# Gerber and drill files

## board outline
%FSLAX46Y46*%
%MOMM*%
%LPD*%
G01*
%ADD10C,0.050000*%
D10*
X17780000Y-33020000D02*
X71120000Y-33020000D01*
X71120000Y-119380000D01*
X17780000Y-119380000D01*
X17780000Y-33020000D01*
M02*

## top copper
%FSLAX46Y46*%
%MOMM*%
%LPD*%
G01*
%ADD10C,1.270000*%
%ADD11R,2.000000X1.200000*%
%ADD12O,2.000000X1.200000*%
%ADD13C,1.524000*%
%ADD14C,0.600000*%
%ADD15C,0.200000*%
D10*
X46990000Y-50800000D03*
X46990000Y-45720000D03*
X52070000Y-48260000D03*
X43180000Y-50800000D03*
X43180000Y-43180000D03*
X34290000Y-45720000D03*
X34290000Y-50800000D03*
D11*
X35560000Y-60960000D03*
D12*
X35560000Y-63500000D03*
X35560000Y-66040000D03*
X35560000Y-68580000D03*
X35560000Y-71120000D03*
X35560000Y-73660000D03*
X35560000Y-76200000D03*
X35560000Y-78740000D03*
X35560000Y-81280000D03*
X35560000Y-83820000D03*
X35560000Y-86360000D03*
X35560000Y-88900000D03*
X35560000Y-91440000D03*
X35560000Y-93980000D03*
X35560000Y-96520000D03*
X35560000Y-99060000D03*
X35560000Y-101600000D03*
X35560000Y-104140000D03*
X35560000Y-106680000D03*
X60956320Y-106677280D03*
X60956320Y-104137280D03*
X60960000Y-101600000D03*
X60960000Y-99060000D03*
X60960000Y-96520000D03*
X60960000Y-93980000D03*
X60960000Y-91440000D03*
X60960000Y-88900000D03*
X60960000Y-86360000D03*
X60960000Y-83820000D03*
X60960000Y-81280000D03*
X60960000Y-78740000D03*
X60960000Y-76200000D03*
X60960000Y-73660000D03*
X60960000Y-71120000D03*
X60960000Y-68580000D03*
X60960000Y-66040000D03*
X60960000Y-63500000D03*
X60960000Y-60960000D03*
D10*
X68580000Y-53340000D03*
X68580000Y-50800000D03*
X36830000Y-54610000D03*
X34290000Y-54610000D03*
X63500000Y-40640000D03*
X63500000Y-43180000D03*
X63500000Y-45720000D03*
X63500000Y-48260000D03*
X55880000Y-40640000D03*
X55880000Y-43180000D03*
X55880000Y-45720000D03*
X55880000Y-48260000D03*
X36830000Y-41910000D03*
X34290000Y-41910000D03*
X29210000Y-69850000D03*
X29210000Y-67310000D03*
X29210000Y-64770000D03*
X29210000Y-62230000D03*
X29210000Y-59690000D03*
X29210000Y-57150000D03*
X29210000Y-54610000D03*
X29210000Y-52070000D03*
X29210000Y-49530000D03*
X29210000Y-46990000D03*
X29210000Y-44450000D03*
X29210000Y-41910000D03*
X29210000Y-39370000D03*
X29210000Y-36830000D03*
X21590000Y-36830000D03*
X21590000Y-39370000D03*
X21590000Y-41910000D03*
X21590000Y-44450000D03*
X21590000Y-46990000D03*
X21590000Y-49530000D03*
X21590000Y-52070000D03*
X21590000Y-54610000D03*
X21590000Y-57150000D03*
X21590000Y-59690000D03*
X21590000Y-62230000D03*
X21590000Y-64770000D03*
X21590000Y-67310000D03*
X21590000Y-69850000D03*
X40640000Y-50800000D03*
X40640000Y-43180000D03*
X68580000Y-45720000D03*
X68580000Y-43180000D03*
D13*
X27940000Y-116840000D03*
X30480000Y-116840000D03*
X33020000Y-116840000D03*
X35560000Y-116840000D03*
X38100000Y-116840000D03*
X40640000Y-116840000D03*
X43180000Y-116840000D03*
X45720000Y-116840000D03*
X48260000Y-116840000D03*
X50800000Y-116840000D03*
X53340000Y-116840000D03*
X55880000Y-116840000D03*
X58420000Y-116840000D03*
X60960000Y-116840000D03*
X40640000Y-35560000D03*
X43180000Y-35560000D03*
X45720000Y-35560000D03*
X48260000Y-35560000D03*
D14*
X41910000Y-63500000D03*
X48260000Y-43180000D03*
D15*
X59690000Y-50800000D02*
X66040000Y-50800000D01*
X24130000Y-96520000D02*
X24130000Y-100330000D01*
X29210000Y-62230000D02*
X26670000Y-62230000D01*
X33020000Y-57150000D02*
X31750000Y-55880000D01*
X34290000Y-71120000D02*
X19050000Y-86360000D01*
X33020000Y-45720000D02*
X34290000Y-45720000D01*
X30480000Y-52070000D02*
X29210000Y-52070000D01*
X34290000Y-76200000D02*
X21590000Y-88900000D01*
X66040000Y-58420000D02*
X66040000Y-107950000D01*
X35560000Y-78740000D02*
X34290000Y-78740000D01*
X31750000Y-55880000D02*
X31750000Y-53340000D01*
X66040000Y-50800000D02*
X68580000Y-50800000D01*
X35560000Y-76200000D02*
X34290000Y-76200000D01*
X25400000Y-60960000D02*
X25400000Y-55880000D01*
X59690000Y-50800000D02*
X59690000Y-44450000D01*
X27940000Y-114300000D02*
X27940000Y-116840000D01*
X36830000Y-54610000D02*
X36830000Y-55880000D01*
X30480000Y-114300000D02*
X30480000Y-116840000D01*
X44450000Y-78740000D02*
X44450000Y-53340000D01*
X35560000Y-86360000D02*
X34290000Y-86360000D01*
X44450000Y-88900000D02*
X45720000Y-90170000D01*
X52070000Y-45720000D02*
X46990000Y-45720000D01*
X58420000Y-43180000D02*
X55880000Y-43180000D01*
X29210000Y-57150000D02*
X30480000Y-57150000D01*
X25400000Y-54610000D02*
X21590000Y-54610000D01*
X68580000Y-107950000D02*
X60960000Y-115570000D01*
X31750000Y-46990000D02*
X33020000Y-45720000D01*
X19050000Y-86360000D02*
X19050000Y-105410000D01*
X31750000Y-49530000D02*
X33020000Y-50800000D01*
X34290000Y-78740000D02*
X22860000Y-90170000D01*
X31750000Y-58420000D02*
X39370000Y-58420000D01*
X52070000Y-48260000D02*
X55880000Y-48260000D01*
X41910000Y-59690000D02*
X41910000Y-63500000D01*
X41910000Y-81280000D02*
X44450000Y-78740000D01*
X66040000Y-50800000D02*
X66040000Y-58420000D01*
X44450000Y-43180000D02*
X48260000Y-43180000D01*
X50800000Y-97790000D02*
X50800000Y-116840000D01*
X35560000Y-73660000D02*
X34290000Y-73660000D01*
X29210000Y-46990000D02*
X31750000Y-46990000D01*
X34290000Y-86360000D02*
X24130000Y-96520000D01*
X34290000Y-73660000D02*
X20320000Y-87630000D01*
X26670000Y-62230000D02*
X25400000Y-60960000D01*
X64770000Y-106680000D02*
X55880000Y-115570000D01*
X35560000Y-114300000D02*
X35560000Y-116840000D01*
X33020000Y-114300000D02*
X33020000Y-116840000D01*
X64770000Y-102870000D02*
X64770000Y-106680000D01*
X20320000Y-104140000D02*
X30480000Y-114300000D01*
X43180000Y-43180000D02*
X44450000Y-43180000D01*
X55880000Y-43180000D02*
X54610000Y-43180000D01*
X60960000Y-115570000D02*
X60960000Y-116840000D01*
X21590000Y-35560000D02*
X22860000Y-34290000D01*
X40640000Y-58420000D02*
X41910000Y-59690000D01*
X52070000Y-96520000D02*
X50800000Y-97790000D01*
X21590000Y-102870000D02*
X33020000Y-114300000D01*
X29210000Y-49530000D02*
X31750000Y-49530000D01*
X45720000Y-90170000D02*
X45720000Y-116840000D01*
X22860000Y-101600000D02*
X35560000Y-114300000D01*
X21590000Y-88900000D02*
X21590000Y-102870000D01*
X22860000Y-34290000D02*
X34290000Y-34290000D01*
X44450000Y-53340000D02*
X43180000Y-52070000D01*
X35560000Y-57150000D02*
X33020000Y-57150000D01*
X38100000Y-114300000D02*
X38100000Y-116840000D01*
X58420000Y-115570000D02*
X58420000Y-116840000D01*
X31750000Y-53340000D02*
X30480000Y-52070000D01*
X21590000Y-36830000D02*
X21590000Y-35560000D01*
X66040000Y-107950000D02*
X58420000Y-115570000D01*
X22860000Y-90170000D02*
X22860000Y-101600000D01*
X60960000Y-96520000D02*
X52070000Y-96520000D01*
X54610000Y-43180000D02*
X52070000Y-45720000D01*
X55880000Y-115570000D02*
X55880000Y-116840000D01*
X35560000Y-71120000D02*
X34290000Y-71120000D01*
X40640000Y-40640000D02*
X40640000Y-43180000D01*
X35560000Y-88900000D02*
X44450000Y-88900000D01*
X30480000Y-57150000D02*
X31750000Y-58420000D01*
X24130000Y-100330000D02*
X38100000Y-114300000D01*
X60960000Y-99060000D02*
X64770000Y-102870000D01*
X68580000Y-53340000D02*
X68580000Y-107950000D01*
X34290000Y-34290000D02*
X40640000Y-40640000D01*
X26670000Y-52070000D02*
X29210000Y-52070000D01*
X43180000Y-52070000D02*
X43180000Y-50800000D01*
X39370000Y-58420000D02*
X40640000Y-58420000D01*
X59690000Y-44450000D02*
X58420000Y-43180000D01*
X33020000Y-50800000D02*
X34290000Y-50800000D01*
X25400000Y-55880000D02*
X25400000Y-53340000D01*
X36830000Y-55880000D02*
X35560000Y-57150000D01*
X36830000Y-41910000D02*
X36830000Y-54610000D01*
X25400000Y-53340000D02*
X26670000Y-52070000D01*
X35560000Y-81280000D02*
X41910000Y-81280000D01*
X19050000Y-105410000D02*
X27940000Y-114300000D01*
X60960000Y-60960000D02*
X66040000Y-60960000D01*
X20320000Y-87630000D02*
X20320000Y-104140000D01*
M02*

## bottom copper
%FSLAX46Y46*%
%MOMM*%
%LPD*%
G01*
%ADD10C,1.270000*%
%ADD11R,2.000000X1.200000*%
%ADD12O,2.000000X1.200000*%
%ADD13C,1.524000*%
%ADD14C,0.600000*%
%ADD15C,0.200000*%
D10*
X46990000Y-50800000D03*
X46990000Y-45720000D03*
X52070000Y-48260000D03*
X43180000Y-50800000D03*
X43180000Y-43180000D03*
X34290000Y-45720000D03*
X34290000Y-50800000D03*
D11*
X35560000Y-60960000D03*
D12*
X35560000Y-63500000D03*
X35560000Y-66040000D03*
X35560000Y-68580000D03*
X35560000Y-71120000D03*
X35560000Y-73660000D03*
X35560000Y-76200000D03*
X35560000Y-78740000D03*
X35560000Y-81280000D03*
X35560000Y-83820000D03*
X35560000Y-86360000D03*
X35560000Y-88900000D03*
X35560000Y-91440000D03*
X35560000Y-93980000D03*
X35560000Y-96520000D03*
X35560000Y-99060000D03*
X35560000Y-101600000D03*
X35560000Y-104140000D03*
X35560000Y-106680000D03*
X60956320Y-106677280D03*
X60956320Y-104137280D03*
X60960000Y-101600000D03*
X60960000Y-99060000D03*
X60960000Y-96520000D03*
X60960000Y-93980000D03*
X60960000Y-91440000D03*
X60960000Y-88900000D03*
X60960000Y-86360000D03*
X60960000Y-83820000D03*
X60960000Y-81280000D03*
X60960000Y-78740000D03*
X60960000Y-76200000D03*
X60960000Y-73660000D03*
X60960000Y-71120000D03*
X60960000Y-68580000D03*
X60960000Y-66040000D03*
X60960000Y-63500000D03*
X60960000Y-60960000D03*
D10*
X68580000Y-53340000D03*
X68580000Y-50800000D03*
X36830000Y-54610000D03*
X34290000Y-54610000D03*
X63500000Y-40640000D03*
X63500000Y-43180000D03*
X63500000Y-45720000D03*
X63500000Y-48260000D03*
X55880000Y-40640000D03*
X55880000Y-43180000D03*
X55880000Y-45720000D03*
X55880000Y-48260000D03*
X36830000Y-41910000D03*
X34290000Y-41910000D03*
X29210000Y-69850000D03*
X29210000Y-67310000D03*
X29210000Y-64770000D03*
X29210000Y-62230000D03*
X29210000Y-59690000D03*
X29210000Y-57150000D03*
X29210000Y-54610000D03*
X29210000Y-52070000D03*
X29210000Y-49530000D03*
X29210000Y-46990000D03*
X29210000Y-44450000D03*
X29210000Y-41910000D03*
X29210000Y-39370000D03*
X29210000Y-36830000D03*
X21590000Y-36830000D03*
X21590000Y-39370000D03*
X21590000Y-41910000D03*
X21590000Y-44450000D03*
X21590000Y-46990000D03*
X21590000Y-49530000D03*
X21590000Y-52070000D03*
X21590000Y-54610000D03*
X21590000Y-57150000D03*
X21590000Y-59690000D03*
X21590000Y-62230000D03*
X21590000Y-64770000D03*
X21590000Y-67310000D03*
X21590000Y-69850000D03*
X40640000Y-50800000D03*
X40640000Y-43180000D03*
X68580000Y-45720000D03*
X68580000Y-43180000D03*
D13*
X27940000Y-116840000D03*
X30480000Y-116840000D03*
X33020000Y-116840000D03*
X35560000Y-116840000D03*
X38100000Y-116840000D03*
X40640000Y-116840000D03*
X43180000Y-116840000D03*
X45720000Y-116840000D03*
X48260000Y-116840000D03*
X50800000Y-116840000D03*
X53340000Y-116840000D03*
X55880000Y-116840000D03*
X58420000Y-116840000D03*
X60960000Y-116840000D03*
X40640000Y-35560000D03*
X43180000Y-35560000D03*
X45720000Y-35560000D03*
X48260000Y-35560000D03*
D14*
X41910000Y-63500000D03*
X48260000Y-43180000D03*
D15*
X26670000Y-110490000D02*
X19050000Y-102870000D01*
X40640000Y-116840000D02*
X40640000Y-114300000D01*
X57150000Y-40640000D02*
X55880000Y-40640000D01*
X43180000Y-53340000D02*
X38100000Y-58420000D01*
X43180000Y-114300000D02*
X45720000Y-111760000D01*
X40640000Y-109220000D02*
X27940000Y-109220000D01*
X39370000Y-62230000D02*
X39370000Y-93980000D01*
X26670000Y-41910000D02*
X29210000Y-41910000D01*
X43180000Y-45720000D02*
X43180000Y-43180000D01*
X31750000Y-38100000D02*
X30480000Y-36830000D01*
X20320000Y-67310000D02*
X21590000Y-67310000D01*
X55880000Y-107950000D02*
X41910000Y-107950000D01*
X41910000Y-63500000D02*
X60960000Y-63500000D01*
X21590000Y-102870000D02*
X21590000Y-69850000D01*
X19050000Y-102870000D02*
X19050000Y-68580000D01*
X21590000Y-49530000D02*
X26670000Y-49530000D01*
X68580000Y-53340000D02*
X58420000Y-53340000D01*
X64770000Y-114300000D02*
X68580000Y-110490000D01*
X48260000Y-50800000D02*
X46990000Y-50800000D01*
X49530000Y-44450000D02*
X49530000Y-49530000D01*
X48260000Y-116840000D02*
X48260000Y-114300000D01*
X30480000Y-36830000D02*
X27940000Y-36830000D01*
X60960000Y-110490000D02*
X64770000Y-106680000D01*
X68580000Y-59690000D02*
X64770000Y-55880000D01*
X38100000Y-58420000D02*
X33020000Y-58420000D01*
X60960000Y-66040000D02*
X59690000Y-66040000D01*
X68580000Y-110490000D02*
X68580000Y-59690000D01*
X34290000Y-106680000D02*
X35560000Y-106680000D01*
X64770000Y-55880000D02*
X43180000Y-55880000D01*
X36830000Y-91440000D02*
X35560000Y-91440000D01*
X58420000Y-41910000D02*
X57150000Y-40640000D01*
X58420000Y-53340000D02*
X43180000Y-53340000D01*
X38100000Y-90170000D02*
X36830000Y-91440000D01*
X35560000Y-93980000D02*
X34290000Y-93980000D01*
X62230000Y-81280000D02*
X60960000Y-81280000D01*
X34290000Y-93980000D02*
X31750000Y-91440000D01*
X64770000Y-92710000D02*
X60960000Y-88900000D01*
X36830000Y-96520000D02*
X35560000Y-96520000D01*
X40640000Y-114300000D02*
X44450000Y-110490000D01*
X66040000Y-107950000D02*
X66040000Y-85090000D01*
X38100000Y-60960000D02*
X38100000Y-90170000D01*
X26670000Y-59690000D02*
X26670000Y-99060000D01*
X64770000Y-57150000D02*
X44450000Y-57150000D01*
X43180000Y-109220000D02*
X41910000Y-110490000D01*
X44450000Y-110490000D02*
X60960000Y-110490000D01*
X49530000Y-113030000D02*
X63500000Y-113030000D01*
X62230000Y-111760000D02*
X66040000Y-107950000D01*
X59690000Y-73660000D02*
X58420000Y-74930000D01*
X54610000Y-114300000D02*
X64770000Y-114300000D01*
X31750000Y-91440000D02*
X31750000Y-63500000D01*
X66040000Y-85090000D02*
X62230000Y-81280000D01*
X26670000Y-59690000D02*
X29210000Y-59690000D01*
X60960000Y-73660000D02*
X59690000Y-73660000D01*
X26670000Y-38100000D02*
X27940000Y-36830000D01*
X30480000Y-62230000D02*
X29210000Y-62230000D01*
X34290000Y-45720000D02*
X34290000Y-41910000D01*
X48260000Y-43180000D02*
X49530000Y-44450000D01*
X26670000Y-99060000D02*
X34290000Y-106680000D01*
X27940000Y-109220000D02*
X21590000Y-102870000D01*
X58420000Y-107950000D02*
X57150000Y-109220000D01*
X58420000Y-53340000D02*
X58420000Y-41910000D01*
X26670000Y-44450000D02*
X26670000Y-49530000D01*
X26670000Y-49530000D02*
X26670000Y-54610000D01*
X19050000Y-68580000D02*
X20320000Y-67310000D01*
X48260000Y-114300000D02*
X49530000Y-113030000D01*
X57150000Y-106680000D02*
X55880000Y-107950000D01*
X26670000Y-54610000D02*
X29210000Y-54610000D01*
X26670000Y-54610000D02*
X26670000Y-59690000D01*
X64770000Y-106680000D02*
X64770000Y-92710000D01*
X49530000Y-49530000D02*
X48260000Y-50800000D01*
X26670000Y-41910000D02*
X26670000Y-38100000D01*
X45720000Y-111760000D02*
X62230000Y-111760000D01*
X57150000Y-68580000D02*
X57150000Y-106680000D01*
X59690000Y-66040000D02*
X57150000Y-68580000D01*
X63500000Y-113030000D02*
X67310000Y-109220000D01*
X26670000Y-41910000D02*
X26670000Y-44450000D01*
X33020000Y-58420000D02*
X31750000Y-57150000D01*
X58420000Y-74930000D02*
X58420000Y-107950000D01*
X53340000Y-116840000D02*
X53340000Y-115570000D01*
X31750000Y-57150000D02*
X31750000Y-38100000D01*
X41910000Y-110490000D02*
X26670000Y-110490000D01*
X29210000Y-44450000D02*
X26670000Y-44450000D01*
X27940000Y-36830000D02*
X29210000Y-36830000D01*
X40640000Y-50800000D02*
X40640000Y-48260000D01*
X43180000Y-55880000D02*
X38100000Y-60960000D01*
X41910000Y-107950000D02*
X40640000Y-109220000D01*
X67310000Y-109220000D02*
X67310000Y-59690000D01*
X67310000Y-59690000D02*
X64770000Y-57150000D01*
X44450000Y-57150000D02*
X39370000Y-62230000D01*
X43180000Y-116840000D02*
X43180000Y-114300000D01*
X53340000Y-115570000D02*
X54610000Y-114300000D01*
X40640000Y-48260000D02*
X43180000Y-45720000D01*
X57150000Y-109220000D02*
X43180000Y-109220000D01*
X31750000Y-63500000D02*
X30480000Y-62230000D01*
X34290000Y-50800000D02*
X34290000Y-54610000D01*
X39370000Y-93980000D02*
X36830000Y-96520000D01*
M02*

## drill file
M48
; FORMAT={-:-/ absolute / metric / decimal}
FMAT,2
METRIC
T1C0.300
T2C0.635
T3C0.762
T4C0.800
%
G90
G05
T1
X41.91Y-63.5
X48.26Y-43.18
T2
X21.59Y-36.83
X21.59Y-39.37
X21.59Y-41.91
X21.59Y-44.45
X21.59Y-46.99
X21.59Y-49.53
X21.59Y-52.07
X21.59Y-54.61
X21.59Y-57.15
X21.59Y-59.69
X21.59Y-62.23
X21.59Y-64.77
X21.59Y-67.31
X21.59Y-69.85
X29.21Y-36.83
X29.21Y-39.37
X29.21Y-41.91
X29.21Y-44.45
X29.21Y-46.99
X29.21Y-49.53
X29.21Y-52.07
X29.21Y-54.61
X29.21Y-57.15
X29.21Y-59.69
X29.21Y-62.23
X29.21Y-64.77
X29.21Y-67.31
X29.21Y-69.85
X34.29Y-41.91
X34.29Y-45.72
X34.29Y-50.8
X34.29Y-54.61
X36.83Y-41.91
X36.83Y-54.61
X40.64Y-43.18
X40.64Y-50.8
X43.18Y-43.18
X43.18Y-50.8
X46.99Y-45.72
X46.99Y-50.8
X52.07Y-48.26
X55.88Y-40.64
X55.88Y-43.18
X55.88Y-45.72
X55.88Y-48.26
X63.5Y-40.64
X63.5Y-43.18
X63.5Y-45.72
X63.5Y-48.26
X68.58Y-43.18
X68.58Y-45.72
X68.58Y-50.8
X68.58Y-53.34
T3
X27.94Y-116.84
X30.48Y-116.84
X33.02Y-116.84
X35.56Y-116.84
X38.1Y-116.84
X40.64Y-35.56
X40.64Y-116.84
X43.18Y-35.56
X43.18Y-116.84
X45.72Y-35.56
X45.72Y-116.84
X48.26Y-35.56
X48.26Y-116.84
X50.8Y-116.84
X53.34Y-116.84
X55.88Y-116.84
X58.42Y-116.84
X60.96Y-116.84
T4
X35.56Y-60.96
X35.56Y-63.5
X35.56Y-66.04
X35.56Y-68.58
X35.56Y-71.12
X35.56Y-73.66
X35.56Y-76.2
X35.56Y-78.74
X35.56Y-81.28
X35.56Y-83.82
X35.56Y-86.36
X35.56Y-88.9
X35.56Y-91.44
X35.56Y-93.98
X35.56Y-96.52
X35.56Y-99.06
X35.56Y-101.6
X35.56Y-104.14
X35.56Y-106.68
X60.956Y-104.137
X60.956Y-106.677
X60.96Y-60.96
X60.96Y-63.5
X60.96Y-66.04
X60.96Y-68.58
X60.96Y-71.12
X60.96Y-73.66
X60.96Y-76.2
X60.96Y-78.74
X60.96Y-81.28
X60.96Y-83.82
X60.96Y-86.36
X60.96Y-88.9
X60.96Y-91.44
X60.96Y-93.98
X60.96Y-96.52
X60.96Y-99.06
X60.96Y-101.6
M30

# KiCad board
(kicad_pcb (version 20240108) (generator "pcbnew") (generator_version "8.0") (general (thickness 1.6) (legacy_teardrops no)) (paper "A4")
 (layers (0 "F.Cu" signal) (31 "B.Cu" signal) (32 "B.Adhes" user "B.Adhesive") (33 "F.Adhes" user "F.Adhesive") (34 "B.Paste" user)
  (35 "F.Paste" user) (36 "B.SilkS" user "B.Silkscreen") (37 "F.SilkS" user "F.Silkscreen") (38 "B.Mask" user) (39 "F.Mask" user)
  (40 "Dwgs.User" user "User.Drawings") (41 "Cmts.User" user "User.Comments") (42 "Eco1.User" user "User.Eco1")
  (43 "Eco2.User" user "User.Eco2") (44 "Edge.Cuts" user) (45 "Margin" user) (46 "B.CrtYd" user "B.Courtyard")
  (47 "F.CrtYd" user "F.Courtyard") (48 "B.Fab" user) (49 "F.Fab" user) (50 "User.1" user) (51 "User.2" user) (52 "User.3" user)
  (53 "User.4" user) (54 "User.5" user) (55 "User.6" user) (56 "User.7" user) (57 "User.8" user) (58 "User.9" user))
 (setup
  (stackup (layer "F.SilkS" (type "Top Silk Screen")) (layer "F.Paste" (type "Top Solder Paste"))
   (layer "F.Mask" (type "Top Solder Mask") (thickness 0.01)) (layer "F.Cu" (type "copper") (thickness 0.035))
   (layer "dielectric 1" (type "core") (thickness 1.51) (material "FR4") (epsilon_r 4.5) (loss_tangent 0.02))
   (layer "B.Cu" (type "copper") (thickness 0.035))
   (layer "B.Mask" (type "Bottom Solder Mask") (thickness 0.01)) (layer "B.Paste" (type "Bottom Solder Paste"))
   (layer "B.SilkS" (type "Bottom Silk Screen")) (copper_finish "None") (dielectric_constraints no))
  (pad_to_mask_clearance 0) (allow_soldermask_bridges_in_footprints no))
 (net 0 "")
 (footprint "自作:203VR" (layer "F.Cu") (at 49.53 48.26 -90)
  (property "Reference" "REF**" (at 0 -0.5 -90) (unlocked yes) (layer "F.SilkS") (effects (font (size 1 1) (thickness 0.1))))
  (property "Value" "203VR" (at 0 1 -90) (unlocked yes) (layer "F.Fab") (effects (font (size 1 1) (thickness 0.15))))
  (pad "1" thru_hole circle (at 2.54 2.54 270) (size 1.27 1.27) (drill 0.635) (layers "*.Cu" "*.Mask") (remove_unused_layers no))
  (pad "2" thru_hole circle (at -2.54 2.54 270) (size 1.27 1.27) (drill 0.635) (layers "*.Cu" "*.Mask") (remove_unused_layers no))
  (pad "3" thru_hole circle (at 0 -2.54 270) (size 1.27 1.27) (drill 0.635) (layers "*.Cu" "*.Mask") (remove_unused_layers no)))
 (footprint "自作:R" (layer "F.Cu") (at 43.18 46.99 -90)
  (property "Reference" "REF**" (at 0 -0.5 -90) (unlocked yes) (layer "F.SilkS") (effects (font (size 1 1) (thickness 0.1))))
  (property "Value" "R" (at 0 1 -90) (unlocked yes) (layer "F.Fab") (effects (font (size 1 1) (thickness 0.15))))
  (pad "1" thru_hole circle (at 3.81 0 270) (size 1.27 1.27) (drill 0.635) (layers "*.Cu" "*.Mask") (remove_unused_layers no))
  (pad "2" thru_hole circle (at -3.81 0 270) (size 1.27 1.27) (drill 0.635) (layers "*.Cu" "*.Mask") (remove_unused_layers no)))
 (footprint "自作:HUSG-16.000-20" (layer "F.Cu") (at 34.29 48.26 90)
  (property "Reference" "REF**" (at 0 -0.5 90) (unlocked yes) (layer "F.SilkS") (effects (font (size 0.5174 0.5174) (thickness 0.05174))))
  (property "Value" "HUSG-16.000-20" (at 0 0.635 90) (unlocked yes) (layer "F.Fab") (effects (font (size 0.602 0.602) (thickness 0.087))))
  (pad "1" thru_hole circle (at 2.54 0 90) (size 1.27 1.27) (drill 0.635) (layers "*.Cu" "*.Mask") (remove_unused_layers no))
  (pad "2" thru_hole circle (at -2.54 0 90) (size 1.27 1.27) (drill 0.635) (layers "*.Cu" "*.Mask") (remove_unused_layers no)))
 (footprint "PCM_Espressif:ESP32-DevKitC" (layer "F.Cu") (at 35.56 60.96)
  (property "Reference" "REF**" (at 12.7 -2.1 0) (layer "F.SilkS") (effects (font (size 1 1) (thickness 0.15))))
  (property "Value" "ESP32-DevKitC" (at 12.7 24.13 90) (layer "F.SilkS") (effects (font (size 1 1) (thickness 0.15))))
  (pad "1" thru_hole rect (at 0 0 270) (size 1.2 2) (drill 0.8) (layers "*.Cu" "*.Mask") (remove_unused_layers no))
  (pad "2" thru_hole oval (at 0 2.54 270) (size 1.2 2) (drill 0.8) (layers "*.Cu" "*.Mask") (remove_unused_layers no))
  (pad "3" thru_hole oval (at 0 5.08 270) (size 1.2 2) (drill 0.8) (layers "*.Cu" "*.Mask") (remove_unused_layers no))
  (pad "4" thru_hole oval (at 0 7.62 270) (size 1.2 2) (drill 0.8) (layers "*.Cu" "*.Mask") (remove_unused_layers no))
  (pad "5" thru_hole oval (at 0 10.16 270) (size 1.2 2) (drill 0.8) (layers "*.Cu" "*.Mask") (remove_unused_layers no))
  (pad "6" thru_hole oval (at 0 12.7 270) (size 1.2 2) (drill 0.8) (layers "*.Cu" "*.Mask") (remove_unused_layers no))
  (pad "7" thru_hole oval (at 0 15.24 270) (size 1.2 2) (drill 0.8) (layers "*.Cu" "*.Mask") (remove_unused_layers no))
  (pad "8" thru_hole oval (at 0 17.78 270) (size 1.2 2) (drill 0.8) (layers "*.Cu" "*.Mask") (remove_unused_layers no))
  (pad "9" thru_hole oval (at 0 20.32 270) (size 1.2 2) (drill 0.8) (layers "*.Cu" "*.Mask") (remove_unused_layers no))
  (pad "10" thru_hole oval (at 0 22.86 270) (size 1.2 2) (drill 0.8) (layers "*.Cu" "*.Mask") (remove_unused_layers no))
  (pad "11" thru_hole oval (at 0 25.4 270) (size 1.2 2) (drill 0.8) (layers "*.Cu" "*.Mask") (remove_unused_layers no))
  (pad "12" thru_hole oval (at 0 27.94 270) (size 1.2 2) (drill 0.8) (layers "*.Cu" "*.Mask") (remove_unused_layers no))
  (pad "13" thru_hole oval (at 0 30.48 270) (size 1.2 2) (drill 0.8) (layers "*.Cu" "*.Mask") (remove_unused_layers no))
  (pad "14" thru_hole oval (at 0 33.02 270) (size 1.2 2) (drill 0.8) (layers "*.Cu" "*.Mask") (remove_unused_layers no))
  (pad "15" thru_hole oval (at 0 35.56 270) (size 1.2 2) (drill 0.8) (layers "*.Cu" "*.Mask") (remove_unused_layers no))
  (pad "16" thru_hole oval (at 0 38.1 270) (size 1.2 2) (drill 0.8) (layers "*.Cu" "*.Mask") (remove_unused_layers no))
  (pad "17" thru_hole oval (at 0 40.64 270) (size 1.2 2) (drill 0.8) (layers "*.Cu" "*.Mask") (remove_unused_layers no))
  (pad "18" thru_hole oval (at 0 43.18 270) (size 1.2 2) (drill 0.8) (layers "*.Cu" "*.Mask") (remove_unused_layers no))
  (pad "19" thru_hole oval (at 0 45.72 270) (size 1.2 2) (drill 0.8) (layers "*.Cu" "*.Mask") (remove_unused_layers no))
  (pad "20" thru_hole oval (at 25.39632 45.71728 270) (size 1.2 2) (drill 0.8) (layers "*.Cu" "*.Mask") (remove_unused_layers no))
  (pad "21" thru_hole oval (at 25.39632 43.17728 270) (size 1.2 2) (drill 0.8) (layers "*.Cu" "*.Mask") (remove_unused_layers no))
  (pad "22" thru_hole oval (at 25.4 40.64 270) (size 1.2 2) (drill 0.8) (layers "*.Cu" "*.Mask") (remove_unused_layers no))
  (pad "23" thru_hole oval (at 25.4 38.1 270) (size 1.2 2) (drill 0.8) (layers "*.Cu" "*.Mask") (remove_unused_layers no))
  (pad "24" thru_hole oval (at 25.4 35.56 270) (size 1.2 2) (drill 0.8) (layers "*.Cu" "*.Mask") (remove_unused_layers no))
  (pad "25" thru_hole oval (at 25.4 33.02 270) (size 1.2 2) (drill 0.8) (layers "*.Cu" "*.Mask") (remove_unused_layers no))
  (pad "26" thru_hole oval (at 25.4 30.48 270) (size 1.2 2) (drill 0.8) (layers "*.Cu" "*.Mask") (remove_unused_layers no))
  (pad "27" thru_hole oval (at 25.4 27.94 270) (size 1.2 2) (drill 0.8) (layers "*.Cu" "*.Mask") (remove_unused_layers no))
  (pad "28" thru_hole oval (at 25.4 25.4 270) (size 1.2 2) (drill 0.8) (layers "*.Cu" "*.Mask") (remove_unused_layers no))
  (pad "29" thru_hole oval (at 25.4 22.86 270) (size 1.2 2) (drill 0.8) (layers "*.Cu" "*.Mask") (remove_unused_layers no))
  (pad "30" thru_hole oval (at 25.4 20.32 270) (size 1.2 2) (drill 0.8) (layers "*.Cu" "*.Mask") (remove_unused_layers no))
  (pad "31" thru_hole oval (at 25.4 17.78 270) (size 1.2 2) (drill 0.8) (layers "*.Cu" "*.Mask") (remove_unused_layers no))
  (pad "32" thru_hole oval (at 25.4 15.24 270) (size 1.2 2) (drill 0.8) (layers "*.Cu" "*.Mask") (remove_unused_layers no))
  (pad "33" thru_hole oval (at 25.4 12.7 270) (size 1.2 2) (drill 0.8) (layers "*.Cu" "*.Mask") (remove_unused_layers no))
  (pad "34" thru_hole oval (at 25.4 10.16 270) (size 1.2 2) (drill 0.8) (layers "*.Cu" "*.Mask") (remove_unused_layers no))
  (pad "35" thru_hole oval (at 25.4 7.62 270) (size 1.2 2) (drill 0.8) (layers "*.Cu" "*.Mask") (remove_unused_layers no))
  (pad "36" thru_hole oval (at 25.4 5.08 270) (size 1.2 2) (drill 0.8) (layers "*.Cu" "*.Mask") (remove_unused_layers no))
  (pad "37" thru_hole oval (at 25.4 2.54 270) (size 1.2 2) (drill 0.8) (layers "*.Cu" "*.Mask") (remove_unused_layers no))
  (pad "38" thru_hole oval (at 25.4 0 270) (size 1.2 2) (drill 0.8) (layers "*.Cu" "*.Mask") (remove_unused_layers no)))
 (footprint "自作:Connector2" (layer "F.Cu") (at 68.58 52.07 90)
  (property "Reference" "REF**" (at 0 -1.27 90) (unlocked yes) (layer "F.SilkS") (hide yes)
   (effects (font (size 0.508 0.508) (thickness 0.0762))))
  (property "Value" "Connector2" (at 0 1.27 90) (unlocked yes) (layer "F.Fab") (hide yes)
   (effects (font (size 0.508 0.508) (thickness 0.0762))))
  (pad "1" thru_hole circle (at -1.27 0 90) (size 1.27 1.27) (drill 0.635) (layers "*.Cu" "*.Mask") (remove_unused_layers no))
  (pad "2" thru_hole circle (at 1.27 0 90) (size 1.27 1.27) (drill 0.635) (layers "*.Cu" "*.Mask") (remove_unused_layers no)))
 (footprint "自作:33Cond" (layer "F.Cu") (at 35.56 54.61)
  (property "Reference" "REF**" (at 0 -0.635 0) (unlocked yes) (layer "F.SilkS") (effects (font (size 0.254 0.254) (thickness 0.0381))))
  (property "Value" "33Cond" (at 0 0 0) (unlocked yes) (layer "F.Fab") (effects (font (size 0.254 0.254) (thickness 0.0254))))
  (pad "1" thru_hole circle (at 1.27 0) (size 1.27 1.27) (drill 0.635) (layers "*.Cu" "*.Mask") (remove_unused_layers no))
  (pad "2" thru_hole circle (at -1.27 0) (size 1.27 1.27) (drill 0.635) (layers "*.Cu" "*.Mask") (remove_unused_layers no)))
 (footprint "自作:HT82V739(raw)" (layer "F.Cu") (at 59.69 44.45)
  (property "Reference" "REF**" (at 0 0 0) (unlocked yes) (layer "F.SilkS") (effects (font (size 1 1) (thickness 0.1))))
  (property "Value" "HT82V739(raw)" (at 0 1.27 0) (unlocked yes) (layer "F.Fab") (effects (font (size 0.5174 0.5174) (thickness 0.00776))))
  (pad "1" thru_hole circle (at 3.81 -3.81) (size 1.27 1.27) (drill 0.635) (layers "*.Cu" "*.Mask") (remove_unused_layers no))
  (pad "2" thru_hole circle (at 3.81 -1.27) (size 1.27 1.27) (drill 0.635) (layers "*.Cu" "*.Mask") (remove_unused_layers no))
  (pad "3" thru_hole circle (at 3.81 1.27) (size 1.27 1.27) (drill 0.635) (layers "*.Cu" "*.Mask") (remove_unused_layers no))
  (pad "4" thru_hole circle (at 3.81 3.81) (size 1.27 1.27) (drill 0.635) (layers "*.Cu" "*.Mask") (remove_unused_layers no))
  (pad "5" thru_hole circle (at -3.81 -3.81) (size 1.27 1.27) (drill 0.635) (layers "*.Cu" "*.Mask") (remove_unused_layers no))
  (pad "6" thru_hole circle (at -3.81 -1.27) (size 1.27 1.27) (drill 0.635) (layers "*.Cu" "*.Mask") (remove_unused_layers no))
  (pad "7" thru_hole circle (at -3.81 1.27) (size 1.27 1.27) (drill 0.635) (layers "*.Cu" "*.Mask") (remove_unused_layers no))
  (pad "8" thru_hole circle (at -3.81 3.81) (size 1.27 1.27) (drill 0.635) (layers "*.Cu" "*.Mask") (remove_unused_layers no)))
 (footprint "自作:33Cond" (layer "F.Cu") (at 35.56 41.91)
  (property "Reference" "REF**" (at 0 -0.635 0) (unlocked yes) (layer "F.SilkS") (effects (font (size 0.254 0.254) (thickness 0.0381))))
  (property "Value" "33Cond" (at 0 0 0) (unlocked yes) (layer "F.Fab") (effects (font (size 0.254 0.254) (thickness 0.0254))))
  (pad "1" thru_hole circle (at 1.27 0) (size 1.27 1.27) (drill 0.635) (layers "*.Cu" "*.Mask") (remove_unused_layers no))
  (pad "2" thru_hole circle (at -1.27 0) (size 1.27 1.27) (drill 0.635) (layers "*.Cu" "*.Mask") (remove_unused_layers no)))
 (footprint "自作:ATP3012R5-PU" (layer "F.Cu") (at 24.13 53.34 90)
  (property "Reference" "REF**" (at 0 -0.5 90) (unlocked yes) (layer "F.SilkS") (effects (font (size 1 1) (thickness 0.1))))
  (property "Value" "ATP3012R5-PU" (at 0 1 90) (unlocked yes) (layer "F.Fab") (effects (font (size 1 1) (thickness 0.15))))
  (pad "1" thru_hole circle (at -16.51 5.08 90) (size 1.27 1.27) (drill 0.635) (layers "*.Cu" "*.Mask") (remove_unused_layers no))
  (pad "2" thru_hole circle (at -13.97 5.08 90) (size 1.27 1.27) (drill 0.635) (layers "*.Cu" "*.Mask") (remove_unused_layers no))
  (pad "3" thru_hole circle (at -11.43 5.08 90) (size 1.27 1.27) (drill 0.635) (layers "*.Cu" "*.Mask") (remove_unused_layers no))
  (pad "4" thru_hole circle (at -8.89 5.08 90) (size 1.27 1.27) (drill 0.635) (layers "*.Cu" "*.Mask") (remove_unused_layers no))
  (pad "5" thru_hole circle (at -6.35 5.08 90) (size 1.27 1.27) (drill 0.635) (layers "*.Cu" "*.Mask") (remove_unused_layers no))
  (pad "6" thru_hole circle (at -3.81 5.08 90) (size 1.27 1.27) (drill 0.635) (layers "*.Cu" "*.Mask") (remove_unused_layers no))
  (pad "7" thru_hole circle (at -1.27 5.08 90) (size 1.27 1.27) (drill 0.635) (layers "*.Cu" "*.Mask") (remove_unused_layers no))
  (pad "8" thru_hole circle (at 1.27 5.08 90) (size 1.27 1.27) (drill 0.635) (layers "*.Cu" "*.Mask") (remove_unused_layers no))
  (pad "9" thru_hole circle (at 3.81 5.08 90) (size 1.27 1.27) (drill 0.635) (layers "*.Cu" "*.Mask") (remove_unused_layers no))
  (pad "10" thru_hole circle (at 6.35 5.08 90) (size 1.27 1.27) (drill 0.635) (layers "*.Cu" "*.Mask") (remove_unused_layers no))
  (pad "11" thru_hole circle (at 8.89 5.08 90) (size 1.27 1.27) (drill 0.635) (layers "*.Cu" "*.Mask") (remove_unused_layers no))
  (pad "12" thru_hole circle (at 11.43 5.08 90) (size 1.27 1.27) (drill 0.635) (layers "*.Cu" "*.Mask") (remove_unused_layers no))
  (pad "13" thru_hole circle (at 13.97 5.08 90) (size 1.27 1.27) (drill 0.635) (layers "*.Cu" "*.Mask") (remove_unused_layers no))
  (pad "14" thru_hole circle (at 16.51 5.08 90) (size 1.27 1.27) (drill 0.635) (layers "*.Cu" "*.Mask") (remove_unused_layers no))
  (pad "15" thru_hole circle (at 16.51 -2.54 90) (size 1.27 1.27) (drill 0.635) (layers "*.Cu" "*.Mask") (remove_unused_layers no))
  (pad "16" thru_hole circle (at 13.97 -2.54 90) (size 1.27 1.27) (drill 0.635) (layers "*.Cu" "*.Mask") (remove_unused_layers no))
  (pad "17" thru_hole circle (at 11.43 -2.54 90) (size 1.27 1.27) (drill 0.635) (layers "*.Cu" "*.Mask") (remove_unused_layers no))
  (pad "18" thru_hole circle (at 8.89 -2.54 90) (size 1.27 1.27) (drill 0.635) (layers "*.Cu" "*.Mask") (remove_unused_layers no))
  (pad "19" thru_hole circle (at 6.35 -2.54 90) (size 1.27 1.27) (drill 0.635) (layers "*.Cu" "*.Mask") (remove_unused_layers no))
  (pad "20" thru_hole circle (at 3.81 -2.54 90) (size 1.27 1.27) (drill 0.635) (layers "*.Cu" "*.Mask") (remove_unused_layers no))
  (pad "21" thru_hole circle (at 1.27 -2.54 90) (size 1.27 1.27) (drill 0.635) (layers "*.Cu" "*.Mask") (remove_unused_layers no))
  (pad "22" thru_hole circle (at -1.27 -2.54 90) (size 1.27 1.27) (drill 0.635) (layers "*.Cu" "*.Mask") (remove_unused_layers no))
  (pad "23" thru_hole circle (at -3.81 -2.54 90) (size 1.27 1.27) (drill 0.635) (layers "*.Cu" "*.Mask") (remove_unused_layers no))
  (pad "24" thru_hole circle (at -6.35 -2.54 90) (size 1.27 1.27) (drill 0.635) (layers "*.Cu" "*.Mask" "F.Adhes") (remove_unused_layers no))
  (pad "25" thru_hole circle (at -8.89 -2.54 90) (size 1.27 1.27) (drill 0.635) (layers "*.Cu" "*.Mask") (remove_unused_layers no))
  (pad "26" thru_hole circle (at -11.43 -2.54 90) (size 1.27 1.27) (drill 0.635) (layers "*.Cu" "*.Mask") (remove_unused_layers no))
  (pad "27" thru_hole circle (at -13.97 -2.54 90) (size 1.27 1.27) (drill 0.635) (layers "*.Cu" "*.Mask") (remove_unused_layers no))
  (pad "28" thru_hole circle (at -16.51 -2.54 90) (size 1.27 1.27) (drill 0.635) (layers "*.Cu" "*.Mask") (remove_unused_layers no)))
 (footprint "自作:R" (layer "F.Cu") (at 40.64 46.99 -90)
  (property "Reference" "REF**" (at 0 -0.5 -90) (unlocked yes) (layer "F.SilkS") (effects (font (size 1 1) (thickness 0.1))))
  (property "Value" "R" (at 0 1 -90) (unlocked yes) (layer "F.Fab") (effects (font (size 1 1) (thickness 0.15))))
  (pad "1" thru_hole circle (at 3.81 0 270) (size 1.27 1.27) (drill 0.635) (layers "*.Cu" "*.Mask") (remove_unused_layers no))
  (pad "2" thru_hole circle (at -3.81 0 270) (size 1.27 1.27) (drill 0.635) (layers "*.Cu" "*.Mask") (remove_unused_layers no)))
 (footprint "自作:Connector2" (layer "F.Cu") (at 68.58 44.45 90)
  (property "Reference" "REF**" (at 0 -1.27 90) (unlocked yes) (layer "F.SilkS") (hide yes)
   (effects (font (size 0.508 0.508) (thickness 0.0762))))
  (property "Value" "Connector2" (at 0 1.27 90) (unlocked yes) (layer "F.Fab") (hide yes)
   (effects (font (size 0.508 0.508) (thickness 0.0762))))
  (pad "1" thru_hole circle (at -1.27 0 90) (size 1.27 1.27) (drill 0.635) (layers "*.Cu" "*.Mask") (remove_unused_layers no))
  (pad "2" thru_hole circle (at 1.27 0 90) (size 1.27 1.27) (drill 0.635) (layers "*.Cu" "*.Mask") (remove_unused_layers no)))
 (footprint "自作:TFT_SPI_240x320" (layer "B.Cu") (at 44.45 76.2 -90)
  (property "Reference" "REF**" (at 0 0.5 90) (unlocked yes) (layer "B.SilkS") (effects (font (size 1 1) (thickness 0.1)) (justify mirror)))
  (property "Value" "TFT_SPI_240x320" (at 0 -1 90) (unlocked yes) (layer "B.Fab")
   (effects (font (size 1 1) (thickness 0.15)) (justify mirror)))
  (pad "1" thru_hole circle (at 40.64 16.51 270) (size 1.524 1.524) (drill 0.762) (layers "*.Cu" "*.Mask") (remove_unused_layers no))
  (pad "2" thru_hole circle (at 40.64 13.97 270) (size 1.524 1.524) (drill 0.762) (layers "*.Cu" "*.Mask") (remove_unused_layers no))
  (pad "3" thru_hole circle (at 40.64 11.43 270) (size 1.524 1.524) (drill 0.762) (layers "*.Cu" "*.Mask") (remove_unused_layers no))
  (pad "4" thru_hole circle (at 40.64 8.89 270) (size 1.524 1.524) (drill 0.762) (layers "*.Cu" "*.Mask") (remove_unused_layers no))
  (pad "5" thru_hole circle (at 40.64 6.35 270) (size 1.524 1.524) (drill 0.762) (layers "*.Cu" "*.Mask") (remove_unused_layers no))
  (pad "6" thru_hole circle (at 40.64 3.81 270) (size 1.524 1.524) (drill 0.762) (layers "*.Cu" "*.Mask") (remove_unused_layers no))
  (pad "7" thru_hole circle (at 40.64 1.27 270) (size 1.524 1.524) (drill 0.762) (layers "*.Cu" "*.Mask") (remove_unused_layers no))
  (pad "8" thru_hole circle (at 40.64 -1.27 270) (size 1.524 1.524) (drill 0.762) (layers "*.Cu" "*.Mask") (remove_unused_layers no))
  (pad "9" thru_hole circle (at 40.64 -3.81 270) (size 1.524 1.524) (drill 0.762) (layers "*.Cu" "*.Mask") (remove_unused_layers no))
  (pad "10" thru_hole circle (at 40.64 -6.35 270) (size 1.524 1.524) (drill 0.762) (layers "*.Cu" "*.Mask") (remove_unused_layers no))
  (pad "11" thru_hole circle (at 40.64 -8.89 270) (size 1.524 1.524) (drill 0.762) (layers "*.Cu" "*.Mask") (remove_unused_layers no))
  (pad "12" thru_hole circle (at 40.64 -11.43 270) (size 1.524 1.524) (drill 0.762) (layers "*.Cu" "*.Mask") (remove_unused_layers no))
  (pad "13" thru_hole circle (at 40.64 -13.97 270) (size 1.524 1.524) (drill 0.762) (layers "*.Cu" "*.Mask") (remove_unused_layers no))
  (pad "14" thru_hole circle (at 40.64 -16.51 270) (size 1.524 1.524) (drill 0.762) (layers "*.Cu" "*.Mask") (remove_unused_layers no))
  (pad "15" thru_hole circle (at -40.64 3.81 270) (size 1.524 1.524) (drill 0.762) (layers "*.Cu" "*.Mask") (remove_unused_layers no))
  (pad "16" thru_hole circle (at -40.64 1.27 270) (size 1.524 1.524) (drill 0.762) (layers "*.Cu" "*.Mask") (remove_unused_layers no))
  (pad "17" thru_hole circle (at -40.64 -1.27 270) (size 1.524 1.524) (drill 0.762) (layers "*.Cu" "*.Mask") (remove_unused_layers no))
  (pad "18" thru_hole circle (at -40.64 -3.81 270) (size 1.524 1.524) (drill 0.762) (layers "*.Cu" "*.Mask") (remove_unused_layers no)))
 (gr_rect (start 17.78 33.02) (end 71.12 119.38) (stroke (width 0.05) (type default)) (fill none) (layer "Edge.Cuts"))
 (segment (start 59.69 50.8) (end 66.04 50.8) (width 0.2) (layer "F.Cu") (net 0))
 (segment (start 24.13 96.52) (end 24.13 100.33) (width 0.2) (layer "F.Cu") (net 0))
 (segment (start 29.21 62.23) (end 26.67 62.23) (width 0.2) (layer "F.Cu") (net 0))
 (segment (start 33.02 57.15) (end 31.75 55.88) (width 0.2) (layer "F.Cu") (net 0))
 (segment (start 34.29 71.12) (end 19.05 86.36) (width 0.2) (layer "F.Cu") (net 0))
 (segment (start 33.02 45.72) (end 34.29 45.72) (width 0.2) (layer "F.Cu") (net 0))
 (segment (start 30.48 52.07) (end 29.21 52.07) (width 0.2) (layer "F.Cu") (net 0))
 (segment (start 34.29 76.2) (end 21.59 88.9) (width 0.2) (layer "F.Cu") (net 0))
 (segment (start 66.04 58.42) (end 66.04 107.95) (width 0.2) (layer "F.Cu") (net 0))
 (segment (start 35.56 78.74) (end 34.29 78.74) (width 0.2) (layer "F.Cu") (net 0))
 (segment (start 31.75 55.88) (end 31.75 53.34) (width 0.2) (layer "F.Cu") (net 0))
 (segment (start 66.04 50.8) (end 68.58 50.8) (width 0.2) (layer "F.Cu") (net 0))
 (segment (start 35.56 76.2) (end 34.29 76.2) (width 0.2) (layer "F.Cu") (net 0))
 (segment (start 25.4 60.96) (end 25.4 55.88) (width 0.2) (layer "F.Cu") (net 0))
 (segment (start 59.69 50.8) (end 59.69 44.45) (width 0.2) (layer "F.Cu") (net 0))
 (segment (start 27.94 114.3) (end 27.94 116.84) (width 0.2) (layer "F.Cu") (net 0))
 (segment (start 36.83 54.61) (end 36.83 55.88) (width 0.2) (layer "F.Cu") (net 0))
 (segment (start 30.48 114.3) (end 30.48 116.84) (width 0.2) (layer "F.Cu") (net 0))
 (segment (start 44.45 78.74) (end 44.45 53.34) (width 0.2) (layer "F.Cu") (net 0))
 (segment (start 35.56 86.36) (end 34.29 86.36) (width 0.2) (layer "F.Cu") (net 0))
 (segment (start 44.45 88.9) (end 45.72 90.17) (width 0.2) (layer "F.Cu") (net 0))
 (segment (start 52.07 45.72) (end 46.99 45.72) (width 0.2) (layer "F.Cu") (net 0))
 (segment (start 58.42 43.18) (end 55.88 43.18) (width 0.2) (layer "F.Cu") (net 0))
 (segment (start 29.21 57.15) (end 30.48 57.15) (width 0.2) (layer "F.Cu") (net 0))
 (segment (start 25.4 54.61) (end 21.59 54.61) (width 0.2) (layer "F.Cu") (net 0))
 (segment (start 68.58 107.95) (end 60.96 115.57) (width 0.2) (layer "F.Cu") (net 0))
 (segment (start 31.75 46.99) (end 33.02 45.72) (width 0.2) (layer "F.Cu") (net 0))
 (segment (start 19.05 86.36) (end 19.05 105.41) (width 0.2) (layer "F.Cu") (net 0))
 (segment (start 31.75 49.53) (end 33.02 50.8) (width 0.2) (layer "F.Cu") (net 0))
 (segment (start 34.29 78.74) (end 22.86 90.17) (width 0.2) (layer "F.Cu") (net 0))
 (segment (start 31.75 58.42) (end 39.37 58.42) (width 0.2) (layer "F.Cu") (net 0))
 (segment (start 52.07 48.26) (end 55.88 48.26) (width 0.2) (layer "F.Cu") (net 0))
 (segment (start 41.91 59.69) (end 41.91 63.5) (width 0.2) (layer "F.Cu") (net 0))
 (segment (start 41.91 81.28) (end 44.45 78.74) (width 0.2) (layer "F.Cu") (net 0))
 (segment (start 66.04 50.8) (end 66.04 58.42) (width 0.2) (layer "F.Cu") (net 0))
 (segment (start 44.45 43.18) (end 48.26 43.18) (width 0.2) (layer "F.Cu") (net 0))
 (segment (start 50.8 97.79) (end 50.8 116.84) (width 0.2) (layer "F.Cu") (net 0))
 (segment (start 35.56 73.66) (end 34.29 73.66) (width 0.2) (layer "F.Cu") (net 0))
 (segment (start 29.21 46.99) (end 31.75 46.99) (width 0.2) (layer "F.Cu") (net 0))
 (segment (start 34.29 86.36) (end 24.13 96.52) (width 0.2) (layer "F.Cu") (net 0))
 (segment (start 34.29 73.66) (end 20.32 87.63) (width 0.2) (layer "F.Cu") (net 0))
 (segment (start 26.67 62.23) (end 25.4 60.96) (width 0.2) (layer "F.Cu") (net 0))
 (segment (start 64.77 106.68) (end 55.88 115.57) (width 0.2) (layer "F.Cu") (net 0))
 (segment (start 35.56 114.3) (end 35.56 116.84) (width 0.2) (layer "F.Cu") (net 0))
 (segment (start 33.02 114.3) (end 33.02 116.84) (width 0.2) (layer "F.Cu") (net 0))
 (segment (start 64.77 102.87) (end 64.77 106.68) (width 0.2) (layer "F.Cu") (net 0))
 (segment (start 20.32 104.14) (end 30.48 114.3) (width 0.2) (layer "F.Cu") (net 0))
 (segment (start 43.18 43.18) (end 44.45 43.18) (width 0.2) (layer "F.Cu") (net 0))
 (segment (start 55.88 43.18) (end 54.61 43.18) (width 0.2) (layer "F.Cu") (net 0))
 (segment (start 60.96 115.57) (end 60.96 116.84) (width 0.2) (layer "F.Cu") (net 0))
 (segment (start 21.59 35.56) (end 22.86 34.29) (width 0.2) (layer "F.Cu") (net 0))
 (segment (start 40.64 58.42) (end 41.91 59.69) (width 0.2) (layer "F.Cu") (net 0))
 (segment (start 52.07 96.52) (end 50.8 97.79) (width 0.2) (layer "F.Cu") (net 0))
 (segment (start 21.59 102.87) (end 33.02 114.3) (width 0.2) (layer "F.Cu") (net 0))
 (segment (start 29.21 49.53) (end 31.75 49.53) (width 0.2) (layer "F.Cu") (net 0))
 (segment (start 45.72 90.17) (end 45.72 116.84) (width 0.2) (layer "F.Cu") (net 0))
 (segment (start 22.86 101.6) (end 35.56 114.3) (width 0.2) (layer "F.Cu") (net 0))
 (segment (start 21.59 88.9) (end 21.59 102.87) (width 0.2) (layer "F.Cu") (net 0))
 (segment (start 22.86 34.29) (end 34.29 34.29) (width 0.2) (layer "F.Cu") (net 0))
 (segment (start 44.45 53.34) (end 43.18 52.07) (width 0.2) (layer "F.Cu") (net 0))
 (segment (start 35.56 57.15) (end 33.02 57.15) (width 0.2) (layer "F.Cu") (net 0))
 (segment (start 38.1 114.3) (end 38.1 116.84) (width 0.2) (layer "F.Cu") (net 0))
 (segment (start 58.42 115.57) (end 58.42 116.84) (width 0.2) (layer "F.Cu") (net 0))
 (segment (start 31.75 53.34) (end 30.48 52.07) (width 0.2) (layer "F.Cu") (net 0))
 (segment (start 21.59 36.83) (end 21.59 35.56) (width 0.2) (layer "F.Cu") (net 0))
 (segment (start 66.04 107.95) (end 58.42 115.57) (width 0.2) (layer "F.Cu") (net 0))
 (segment (start 22.86 90.17) (end 22.86 101.6) (width 0.2) (layer "F.Cu") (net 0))
 (segment (start 60.96 96.52) (end 52.07 96.52) (width 0.2) (layer "F.Cu") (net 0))
 (segment (start 54.61 43.18) (end 52.07 45.72) (width 0.2) (layer "F.Cu") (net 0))
 (segment (start 55.88 115.57) (end 55.88 116.84) (width 0.2) (layer "F.Cu") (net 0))
 (segment (start 35.56 71.12) (end 34.29 71.12) (width 0.2) (layer "F.Cu") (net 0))
 (segment (start 40.64 40.64) (end 40.64 43.18) (width 0.2) (layer "F.Cu") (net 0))
 (segment (start 35.56 88.9) (end 44.45 88.9) (width 0.2) (layer "F.Cu") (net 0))
 (segment (start 30.48 57.15) (end 31.75 58.42) (width 0.2) (layer "F.Cu") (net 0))
 (segment (start 24.13 100.33) (end 38.1 114.3) (width 0.2) (layer "F.Cu") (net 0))
 (segment (start 60.96 99.06) (end 64.77 102.87) (width 0.2) (layer "F.Cu") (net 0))
 (segment (start 68.58 53.34) (end 68.58 107.95) (width 0.2) (layer "F.Cu") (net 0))
 (segment (start 34.29 34.29) (end 40.64 40.64) (width 0.2) (layer "F.Cu") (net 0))
 (segment (start 26.67 52.07) (end 29.21 52.07) (width 0.2) (layer "F.Cu") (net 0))
 (segment (start 43.18 52.07) (end 43.18 50.8) (width 0.2) (layer "F.Cu") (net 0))
 (segment (start 39.37 58.42) (end 40.64 58.42) (width 0.2) (layer "F.Cu") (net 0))
 (segment (start 59.69 44.45) (end 58.42 43.18) (width 0.2) (layer "F.Cu") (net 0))
 (segment (start 33.02 50.8) (end 34.29 50.8) (width 0.2) (layer "F.Cu") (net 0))
 (segment (start 25.4 55.88) (end 25.4 53.34) (width 0.2) (layer "F.Cu") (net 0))
 (segment (start 36.83 55.88) (end 35.56 57.15) (width 0.2) (layer "F.Cu") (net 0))
 (segment (start 36.83 41.91) (end 36.83 54.61) (width 0.2) (layer "F.Cu") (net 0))
 (segment (start 25.4 53.34) (end 26.67 52.07) (width 0.2) (layer "F.Cu") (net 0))
 (segment (start 35.56 81.28) (end 41.91 81.28) (width 0.2) (layer "F.Cu") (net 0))
 (segment (start 19.05 105.41) (end 27.94 114.3) (width 0.2) (layer "F.Cu") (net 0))
 (segment (start 60.96 60.96) (end 66.04 60.96) (width 0.2) (layer "F.Cu") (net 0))
 (segment (start 20.32 87.63) (end 20.32 104.14) (width 0.2) (layer "F.Cu") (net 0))
 (via (at 41.91 63.5) (size 0.6) (drill 0.3) (layers "F.Cu" "B.Cu") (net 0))
 (via (at 48.26 43.18) (size 0.6) (drill 0.3) (layers "F.Cu" "B.Cu") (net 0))
 (segment (start 26.67 110.49) (end 19.05 102.87) (width 0.2) (layer "B.Cu") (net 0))
 (segment (start 40.64 116.84) (end 40.64 114.3) (width 0.2) (layer "B.Cu") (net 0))
 (segment (start 57.15 40.64) (end 55.88 40.64) (width 0.2) (layer "B.Cu") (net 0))
 (segment (start 43.18 53.34) (end 38.1 58.42) (width 0.2) (layer "B.Cu") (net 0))
 (segment (start 43.18 114.3) (end 45.72 111.76) (width 0.2) (layer "B.Cu") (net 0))
 (segment (start 40.64 109.22) (end 27.94 109.22) (width 0.2) (layer "B.Cu") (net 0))
 (segment (start 39.37 62.23) (end 39.37 93.98) (width 0.2) (layer "B.Cu") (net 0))
 (segment (start 26.67 41.91) (end 29.21 41.91) (width 0.2) (layer "B.Cu") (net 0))
 (segment (start 43.18 45.72) (end 43.18 43.18) (width 0.2) (layer "B.Cu") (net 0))
 (segment (start 31.75 38.1) (end 30.48 36.83) (width 0.2) (layer "B.Cu") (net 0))
 (segment (start 20.32 67.31) (end 21.59 67.31) (width 0.2) (layer "B.Cu") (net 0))
 (segment (start 55.88 107.95) (end 41.91 107.95) (width 0.2) (layer "B.Cu") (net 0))
 (segment (start 41.91 63.5) (end 60.96 63.5) (width 0.2) (layer "B.Cu") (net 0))
 (segment (start 21.59 102.87) (end 21.59 69.85) (width 0.2) (layer "B.Cu") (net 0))
 (segment (start 19.05 102.87) (end 19.05 68.58) (width 0.2) (layer "B.Cu") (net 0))
 (segment (start 21.59 49.53) (end 26.67 49.53) (width 0.2) (layer "B.Cu") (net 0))
 (segment (start 68.58 53.34) (end 58.42 53.34) (width 0.2) (layer "B.Cu") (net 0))
 (segment (start 64.77 114.3) (end 68.58 110.49) (width 0.2) (layer "B.Cu") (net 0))
 (segment (start 48.26 50.8) (end 46.99 50.8) (width 0.2) (layer "B.Cu") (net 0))
 (segment (start 49.53 44.45) (end 49.53 49.53) (width 0.2) (layer "B.Cu") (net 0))
 (segment (start 48.26 116.84) (end 48.26 114.3) (width 0.2) (layer "B.Cu") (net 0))
 (segment (start 30.48 36.83) (end 27.94 36.83) (width 0.2) (layer "B.Cu") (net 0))
 (segment (start 60.96 110.49) (end 64.77 106.68) (width 0.2) (layer "B.Cu") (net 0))
 (segment (start 68.58 59.69) (end 64.77 55.88) (width 0.2) (layer "B.Cu") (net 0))
 (segment (start 38.1 58.42) (end 33.02 58.42) (width 0.2) (layer "B.Cu") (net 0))
 (segment (start 60.96 66.04) (end 59.69 66.04) (width 0.2) (layer "B.Cu") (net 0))
 (segment (start 68.58 110.49) (end 68.58 59.69) (width 0.2) (layer "B.Cu") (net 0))
 (segment (start 34.29 106.68) (end 35.56 106.68) (width 0.2) (layer "B.Cu") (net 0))
 (segment (start 64.77 55.88) (end 43.18 55.88) (width 0.2) (layer "B.Cu") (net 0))
 (segment (start 36.83 91.44) (end 35.56 91.44) (width 0.2) (layer "B.Cu") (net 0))
 (segment (start 58.42 41.91) (end 57.15 40.64) (width 0.2) (layer "B.Cu") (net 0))
 (segment (start 58.42 53.34) (end 43.18 53.34) (width 0.2) (layer "B.Cu") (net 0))
 (segment (start 38.1 90.17) (end 36.83 91.44) (width 0.2) (layer "B.Cu") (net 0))
 (segment (start 35.56 93.98) (end 34.29 93.98) (width 0.2) (layer "B.Cu") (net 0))
 (segment (start 62.23 81.28) (end 60.96 81.28) (width 0.2) (layer "B.Cu") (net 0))
 (segment (start 34.29 93.98) (end 31.75 91.44) (width 0.2) (layer "B.Cu") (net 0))
 (segment (start 64.77 92.71) (end 60.96 88.9) (width 0.2) (layer "B.Cu") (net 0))
 (segment (start 36.83 96.52) (end 35.56 96.52) (width 0.2) (layer "B.Cu") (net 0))
 (segment (start 40.64 114.3) (end 44.45 110.49) (width 0.2) (layer "B.Cu") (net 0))
 (segment (start 66.04 107.95) (end 66.04 85.09) (width 0.2) (layer "B.Cu") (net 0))
 (segment (start 38.1 60.96) (end 38.1 90.17) (width 0.2) (layer "B.Cu") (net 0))
 (segment (start 26.67 59.69) (end 26.67 99.06) (width 0.2) (layer "B.Cu") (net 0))
 (segment (start 64.77 57.15) (end 44.45 57.15) (width 0.2) (layer "B.Cu") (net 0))
 (segment (start 43.18 109.22) (end 41.91 110.49) (width 0.2) (layer "B.Cu") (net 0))
 (segment (start 44.45 110.49) (end 60.96 110.49) (width 0.2) (layer "B.Cu") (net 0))
 (segment (start 49.53 113.03) (end 63.5 113.03) (width 0.2) (layer "B.Cu") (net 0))
 (segment (start 62.23 111.76) (end 66.04 107.95) (width 0.2) (layer "B.Cu") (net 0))
 (segment (start 59.69 73.66) (end 58.42 74.93) (width 0.2) (layer "B.Cu") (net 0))
 (segment (start 54.61 114.3) (end 64.77 114.3) (width 0.2) (layer "B.Cu") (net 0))
 (segment (start 31.75 91.44) (end 31.75 63.5) (width 0.2) (layer "B.Cu") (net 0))
 (segment (start 66.04 85.09) (end 62.23 81.28) (width 0.2) (layer "B.Cu") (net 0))
 (segment (start 26.67 59.69) (end 29.21 59.69) (width 0.2) (layer "B.Cu") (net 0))
 (segment (start 60.96 73.66) (end 59.69 73.66) (width 0.2) (layer "B.Cu") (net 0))
 (segment (start 26.67 38.1) (end 27.94 36.83) (width 0.2) (layer "B.Cu") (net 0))
 (segment (start 30.48 62.23) (end 29.21 62.23) (width 0.2) (layer "B.Cu") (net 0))
 (segment (start 34.29 45.72) (end 34.29 41.91) (width 0.2) (layer "B.Cu") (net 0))
 (segment (start 48.26 43.18) (end 49.53 44.45) (width 0.2) (layer "B.Cu") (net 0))
 (segment (start 26.67 99.06) (end 34.29 106.68) (width 0.2) (layer "B.Cu") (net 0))
 (segment (start 27.94 109.22) (end 21.59 102.87) (width 0.2) (layer "B.Cu") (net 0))
 (segment (start 58.42 107.95) (end 57.15 109.22) (width 0.2) (layer "B.Cu") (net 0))
 (segment (start 58.42 53.34) (end 58.42 41.91) (width 0.2) (layer "B.Cu") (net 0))
 (segment (start 26.67 44.45) (end 26.67 49.53) (width 0.2) (layer "B.Cu") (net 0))
 (segment (start 26.67 49.53) (end 26.67 54.61) (width 0.2) (layer "B.Cu") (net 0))
 (segment (start 19.05 68.58) (end 20.32 67.31) (width 0.2) (layer "B.Cu") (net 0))
 (segment (start 48.26 114.3) (end 49.53 113.03) (width 0.2) (layer "B.Cu") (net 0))
 (segment (start 57.15 106.68) (end 55.88 107.95) (width 0.2) (layer "B.Cu") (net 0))
 (segment (start 26.67 54.61) (end 29.21 54.61) (width 0.2) (layer "B.Cu") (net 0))
 (segment (start 26.67 54.61) (end 26.67 59.69) (width 0.2) (layer "B.Cu") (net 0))
 (segment (start 64.77 106.68) (end 64.77 92.71) (width 0.2) (layer "B.Cu") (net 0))
 (segment (start 49.53 49.53) (end 48.26 50.8) (width 0.2) (layer "B.Cu") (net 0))
 (segment (start 26.67 41.91) (end 26.67 38.1) (width 0.2) (layer "B.Cu") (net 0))
 (segment (start 45.72 111.76) (end 62.23 111.76) (width 0.2) (layer "B.Cu") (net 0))
 (segment (start 57.15 68.58) (end 57.15 106.68) (width 0.2) (layer "B.Cu") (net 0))
 (segment (start 59.69 66.04) (end 57.15 68.58) (width 0.2) (layer "B.Cu") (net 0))
 (segment (start 63.5 113.03) (end 67.31 109.22) (width 0.2) (layer "B.Cu") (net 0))
 (segment (start 26.67 41.91) (end 26.67 44.45) (width 0.2) (layer "B.Cu") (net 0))
 (segment (start 33.02 58.42) (end 31.75 57.15) (width 0.2) (layer "B.Cu") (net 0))
 (segment (start 58.42 74.93) (end 58.42 107.95) (width 0.2) (layer "B.Cu") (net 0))
 (segment (start 53.34 116.84) (end 53.34 115.57) (width 0.2) (layer "B.Cu") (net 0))
 (segment (start 31.75 57.15) (end 31.75 38.1) (width 0.2) (layer "B.Cu") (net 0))
 (segment (start 41.91 110.49) (end 26.67 110.49) (width 0.2) (layer "B.Cu") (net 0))
 (segment (start 29.21 44.45) (end 26.67 44.45) (width 0.2) (layer "B.Cu") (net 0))
 (segment (start 27.94 36.83) (end 29.21 36.83) (width 0.2) (layer "B.Cu") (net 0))
 (segment (start 40.64 50.8) (end 40.64 48.26) (width 0.2) (layer "B.Cu") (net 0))
 (segment (start 43.18 55.88) (end 38.1 60.96) (width 0.2) (layer "B.Cu") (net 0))
 (segment (start 41.91 107.95) (end 40.64 109.22) (width 0.2) (layer "B.Cu") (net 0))
 (segment (start 67.31 109.22) (end 67.31 59.69) (width 0.2) (layer "B.Cu") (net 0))
 (segment (start 67.31 59.69) (end 64.77 57.15) (width 0.2) (layer "B.Cu") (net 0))
 (segment (start 44.45 57.15) (end 39.37 62.23) (width 0.2) (layer "B.Cu") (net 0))
 (segment (start 43.18 116.84) (end 43.18 114.3) (width 0.2) (layer "B.Cu") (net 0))
 (segment (start 53.34 115.57) (end 54.61 114.3) (width 0.2) (layer "B.Cu") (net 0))
 (segment (start 40.64 48.26) (end 43.18 45.72) (width 0.2) (layer "B.Cu") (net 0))
 (segment (start 57.15 109.22) (end 43.18 109.22) (width 0.2) (layer "B.Cu") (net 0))
 (segment (start 31.75 63.5) (end 30.48 62.23) (width 0.2) (layer "B.Cu") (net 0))
 (segment (start 34.29 50.8) (end 34.29 54.61) (width 0.2) (layer "B.Cu") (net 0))
 (segment (start 39.37 93.98) (end 36.83 96.52) (width 0.2) (layer "B.Cu") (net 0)))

